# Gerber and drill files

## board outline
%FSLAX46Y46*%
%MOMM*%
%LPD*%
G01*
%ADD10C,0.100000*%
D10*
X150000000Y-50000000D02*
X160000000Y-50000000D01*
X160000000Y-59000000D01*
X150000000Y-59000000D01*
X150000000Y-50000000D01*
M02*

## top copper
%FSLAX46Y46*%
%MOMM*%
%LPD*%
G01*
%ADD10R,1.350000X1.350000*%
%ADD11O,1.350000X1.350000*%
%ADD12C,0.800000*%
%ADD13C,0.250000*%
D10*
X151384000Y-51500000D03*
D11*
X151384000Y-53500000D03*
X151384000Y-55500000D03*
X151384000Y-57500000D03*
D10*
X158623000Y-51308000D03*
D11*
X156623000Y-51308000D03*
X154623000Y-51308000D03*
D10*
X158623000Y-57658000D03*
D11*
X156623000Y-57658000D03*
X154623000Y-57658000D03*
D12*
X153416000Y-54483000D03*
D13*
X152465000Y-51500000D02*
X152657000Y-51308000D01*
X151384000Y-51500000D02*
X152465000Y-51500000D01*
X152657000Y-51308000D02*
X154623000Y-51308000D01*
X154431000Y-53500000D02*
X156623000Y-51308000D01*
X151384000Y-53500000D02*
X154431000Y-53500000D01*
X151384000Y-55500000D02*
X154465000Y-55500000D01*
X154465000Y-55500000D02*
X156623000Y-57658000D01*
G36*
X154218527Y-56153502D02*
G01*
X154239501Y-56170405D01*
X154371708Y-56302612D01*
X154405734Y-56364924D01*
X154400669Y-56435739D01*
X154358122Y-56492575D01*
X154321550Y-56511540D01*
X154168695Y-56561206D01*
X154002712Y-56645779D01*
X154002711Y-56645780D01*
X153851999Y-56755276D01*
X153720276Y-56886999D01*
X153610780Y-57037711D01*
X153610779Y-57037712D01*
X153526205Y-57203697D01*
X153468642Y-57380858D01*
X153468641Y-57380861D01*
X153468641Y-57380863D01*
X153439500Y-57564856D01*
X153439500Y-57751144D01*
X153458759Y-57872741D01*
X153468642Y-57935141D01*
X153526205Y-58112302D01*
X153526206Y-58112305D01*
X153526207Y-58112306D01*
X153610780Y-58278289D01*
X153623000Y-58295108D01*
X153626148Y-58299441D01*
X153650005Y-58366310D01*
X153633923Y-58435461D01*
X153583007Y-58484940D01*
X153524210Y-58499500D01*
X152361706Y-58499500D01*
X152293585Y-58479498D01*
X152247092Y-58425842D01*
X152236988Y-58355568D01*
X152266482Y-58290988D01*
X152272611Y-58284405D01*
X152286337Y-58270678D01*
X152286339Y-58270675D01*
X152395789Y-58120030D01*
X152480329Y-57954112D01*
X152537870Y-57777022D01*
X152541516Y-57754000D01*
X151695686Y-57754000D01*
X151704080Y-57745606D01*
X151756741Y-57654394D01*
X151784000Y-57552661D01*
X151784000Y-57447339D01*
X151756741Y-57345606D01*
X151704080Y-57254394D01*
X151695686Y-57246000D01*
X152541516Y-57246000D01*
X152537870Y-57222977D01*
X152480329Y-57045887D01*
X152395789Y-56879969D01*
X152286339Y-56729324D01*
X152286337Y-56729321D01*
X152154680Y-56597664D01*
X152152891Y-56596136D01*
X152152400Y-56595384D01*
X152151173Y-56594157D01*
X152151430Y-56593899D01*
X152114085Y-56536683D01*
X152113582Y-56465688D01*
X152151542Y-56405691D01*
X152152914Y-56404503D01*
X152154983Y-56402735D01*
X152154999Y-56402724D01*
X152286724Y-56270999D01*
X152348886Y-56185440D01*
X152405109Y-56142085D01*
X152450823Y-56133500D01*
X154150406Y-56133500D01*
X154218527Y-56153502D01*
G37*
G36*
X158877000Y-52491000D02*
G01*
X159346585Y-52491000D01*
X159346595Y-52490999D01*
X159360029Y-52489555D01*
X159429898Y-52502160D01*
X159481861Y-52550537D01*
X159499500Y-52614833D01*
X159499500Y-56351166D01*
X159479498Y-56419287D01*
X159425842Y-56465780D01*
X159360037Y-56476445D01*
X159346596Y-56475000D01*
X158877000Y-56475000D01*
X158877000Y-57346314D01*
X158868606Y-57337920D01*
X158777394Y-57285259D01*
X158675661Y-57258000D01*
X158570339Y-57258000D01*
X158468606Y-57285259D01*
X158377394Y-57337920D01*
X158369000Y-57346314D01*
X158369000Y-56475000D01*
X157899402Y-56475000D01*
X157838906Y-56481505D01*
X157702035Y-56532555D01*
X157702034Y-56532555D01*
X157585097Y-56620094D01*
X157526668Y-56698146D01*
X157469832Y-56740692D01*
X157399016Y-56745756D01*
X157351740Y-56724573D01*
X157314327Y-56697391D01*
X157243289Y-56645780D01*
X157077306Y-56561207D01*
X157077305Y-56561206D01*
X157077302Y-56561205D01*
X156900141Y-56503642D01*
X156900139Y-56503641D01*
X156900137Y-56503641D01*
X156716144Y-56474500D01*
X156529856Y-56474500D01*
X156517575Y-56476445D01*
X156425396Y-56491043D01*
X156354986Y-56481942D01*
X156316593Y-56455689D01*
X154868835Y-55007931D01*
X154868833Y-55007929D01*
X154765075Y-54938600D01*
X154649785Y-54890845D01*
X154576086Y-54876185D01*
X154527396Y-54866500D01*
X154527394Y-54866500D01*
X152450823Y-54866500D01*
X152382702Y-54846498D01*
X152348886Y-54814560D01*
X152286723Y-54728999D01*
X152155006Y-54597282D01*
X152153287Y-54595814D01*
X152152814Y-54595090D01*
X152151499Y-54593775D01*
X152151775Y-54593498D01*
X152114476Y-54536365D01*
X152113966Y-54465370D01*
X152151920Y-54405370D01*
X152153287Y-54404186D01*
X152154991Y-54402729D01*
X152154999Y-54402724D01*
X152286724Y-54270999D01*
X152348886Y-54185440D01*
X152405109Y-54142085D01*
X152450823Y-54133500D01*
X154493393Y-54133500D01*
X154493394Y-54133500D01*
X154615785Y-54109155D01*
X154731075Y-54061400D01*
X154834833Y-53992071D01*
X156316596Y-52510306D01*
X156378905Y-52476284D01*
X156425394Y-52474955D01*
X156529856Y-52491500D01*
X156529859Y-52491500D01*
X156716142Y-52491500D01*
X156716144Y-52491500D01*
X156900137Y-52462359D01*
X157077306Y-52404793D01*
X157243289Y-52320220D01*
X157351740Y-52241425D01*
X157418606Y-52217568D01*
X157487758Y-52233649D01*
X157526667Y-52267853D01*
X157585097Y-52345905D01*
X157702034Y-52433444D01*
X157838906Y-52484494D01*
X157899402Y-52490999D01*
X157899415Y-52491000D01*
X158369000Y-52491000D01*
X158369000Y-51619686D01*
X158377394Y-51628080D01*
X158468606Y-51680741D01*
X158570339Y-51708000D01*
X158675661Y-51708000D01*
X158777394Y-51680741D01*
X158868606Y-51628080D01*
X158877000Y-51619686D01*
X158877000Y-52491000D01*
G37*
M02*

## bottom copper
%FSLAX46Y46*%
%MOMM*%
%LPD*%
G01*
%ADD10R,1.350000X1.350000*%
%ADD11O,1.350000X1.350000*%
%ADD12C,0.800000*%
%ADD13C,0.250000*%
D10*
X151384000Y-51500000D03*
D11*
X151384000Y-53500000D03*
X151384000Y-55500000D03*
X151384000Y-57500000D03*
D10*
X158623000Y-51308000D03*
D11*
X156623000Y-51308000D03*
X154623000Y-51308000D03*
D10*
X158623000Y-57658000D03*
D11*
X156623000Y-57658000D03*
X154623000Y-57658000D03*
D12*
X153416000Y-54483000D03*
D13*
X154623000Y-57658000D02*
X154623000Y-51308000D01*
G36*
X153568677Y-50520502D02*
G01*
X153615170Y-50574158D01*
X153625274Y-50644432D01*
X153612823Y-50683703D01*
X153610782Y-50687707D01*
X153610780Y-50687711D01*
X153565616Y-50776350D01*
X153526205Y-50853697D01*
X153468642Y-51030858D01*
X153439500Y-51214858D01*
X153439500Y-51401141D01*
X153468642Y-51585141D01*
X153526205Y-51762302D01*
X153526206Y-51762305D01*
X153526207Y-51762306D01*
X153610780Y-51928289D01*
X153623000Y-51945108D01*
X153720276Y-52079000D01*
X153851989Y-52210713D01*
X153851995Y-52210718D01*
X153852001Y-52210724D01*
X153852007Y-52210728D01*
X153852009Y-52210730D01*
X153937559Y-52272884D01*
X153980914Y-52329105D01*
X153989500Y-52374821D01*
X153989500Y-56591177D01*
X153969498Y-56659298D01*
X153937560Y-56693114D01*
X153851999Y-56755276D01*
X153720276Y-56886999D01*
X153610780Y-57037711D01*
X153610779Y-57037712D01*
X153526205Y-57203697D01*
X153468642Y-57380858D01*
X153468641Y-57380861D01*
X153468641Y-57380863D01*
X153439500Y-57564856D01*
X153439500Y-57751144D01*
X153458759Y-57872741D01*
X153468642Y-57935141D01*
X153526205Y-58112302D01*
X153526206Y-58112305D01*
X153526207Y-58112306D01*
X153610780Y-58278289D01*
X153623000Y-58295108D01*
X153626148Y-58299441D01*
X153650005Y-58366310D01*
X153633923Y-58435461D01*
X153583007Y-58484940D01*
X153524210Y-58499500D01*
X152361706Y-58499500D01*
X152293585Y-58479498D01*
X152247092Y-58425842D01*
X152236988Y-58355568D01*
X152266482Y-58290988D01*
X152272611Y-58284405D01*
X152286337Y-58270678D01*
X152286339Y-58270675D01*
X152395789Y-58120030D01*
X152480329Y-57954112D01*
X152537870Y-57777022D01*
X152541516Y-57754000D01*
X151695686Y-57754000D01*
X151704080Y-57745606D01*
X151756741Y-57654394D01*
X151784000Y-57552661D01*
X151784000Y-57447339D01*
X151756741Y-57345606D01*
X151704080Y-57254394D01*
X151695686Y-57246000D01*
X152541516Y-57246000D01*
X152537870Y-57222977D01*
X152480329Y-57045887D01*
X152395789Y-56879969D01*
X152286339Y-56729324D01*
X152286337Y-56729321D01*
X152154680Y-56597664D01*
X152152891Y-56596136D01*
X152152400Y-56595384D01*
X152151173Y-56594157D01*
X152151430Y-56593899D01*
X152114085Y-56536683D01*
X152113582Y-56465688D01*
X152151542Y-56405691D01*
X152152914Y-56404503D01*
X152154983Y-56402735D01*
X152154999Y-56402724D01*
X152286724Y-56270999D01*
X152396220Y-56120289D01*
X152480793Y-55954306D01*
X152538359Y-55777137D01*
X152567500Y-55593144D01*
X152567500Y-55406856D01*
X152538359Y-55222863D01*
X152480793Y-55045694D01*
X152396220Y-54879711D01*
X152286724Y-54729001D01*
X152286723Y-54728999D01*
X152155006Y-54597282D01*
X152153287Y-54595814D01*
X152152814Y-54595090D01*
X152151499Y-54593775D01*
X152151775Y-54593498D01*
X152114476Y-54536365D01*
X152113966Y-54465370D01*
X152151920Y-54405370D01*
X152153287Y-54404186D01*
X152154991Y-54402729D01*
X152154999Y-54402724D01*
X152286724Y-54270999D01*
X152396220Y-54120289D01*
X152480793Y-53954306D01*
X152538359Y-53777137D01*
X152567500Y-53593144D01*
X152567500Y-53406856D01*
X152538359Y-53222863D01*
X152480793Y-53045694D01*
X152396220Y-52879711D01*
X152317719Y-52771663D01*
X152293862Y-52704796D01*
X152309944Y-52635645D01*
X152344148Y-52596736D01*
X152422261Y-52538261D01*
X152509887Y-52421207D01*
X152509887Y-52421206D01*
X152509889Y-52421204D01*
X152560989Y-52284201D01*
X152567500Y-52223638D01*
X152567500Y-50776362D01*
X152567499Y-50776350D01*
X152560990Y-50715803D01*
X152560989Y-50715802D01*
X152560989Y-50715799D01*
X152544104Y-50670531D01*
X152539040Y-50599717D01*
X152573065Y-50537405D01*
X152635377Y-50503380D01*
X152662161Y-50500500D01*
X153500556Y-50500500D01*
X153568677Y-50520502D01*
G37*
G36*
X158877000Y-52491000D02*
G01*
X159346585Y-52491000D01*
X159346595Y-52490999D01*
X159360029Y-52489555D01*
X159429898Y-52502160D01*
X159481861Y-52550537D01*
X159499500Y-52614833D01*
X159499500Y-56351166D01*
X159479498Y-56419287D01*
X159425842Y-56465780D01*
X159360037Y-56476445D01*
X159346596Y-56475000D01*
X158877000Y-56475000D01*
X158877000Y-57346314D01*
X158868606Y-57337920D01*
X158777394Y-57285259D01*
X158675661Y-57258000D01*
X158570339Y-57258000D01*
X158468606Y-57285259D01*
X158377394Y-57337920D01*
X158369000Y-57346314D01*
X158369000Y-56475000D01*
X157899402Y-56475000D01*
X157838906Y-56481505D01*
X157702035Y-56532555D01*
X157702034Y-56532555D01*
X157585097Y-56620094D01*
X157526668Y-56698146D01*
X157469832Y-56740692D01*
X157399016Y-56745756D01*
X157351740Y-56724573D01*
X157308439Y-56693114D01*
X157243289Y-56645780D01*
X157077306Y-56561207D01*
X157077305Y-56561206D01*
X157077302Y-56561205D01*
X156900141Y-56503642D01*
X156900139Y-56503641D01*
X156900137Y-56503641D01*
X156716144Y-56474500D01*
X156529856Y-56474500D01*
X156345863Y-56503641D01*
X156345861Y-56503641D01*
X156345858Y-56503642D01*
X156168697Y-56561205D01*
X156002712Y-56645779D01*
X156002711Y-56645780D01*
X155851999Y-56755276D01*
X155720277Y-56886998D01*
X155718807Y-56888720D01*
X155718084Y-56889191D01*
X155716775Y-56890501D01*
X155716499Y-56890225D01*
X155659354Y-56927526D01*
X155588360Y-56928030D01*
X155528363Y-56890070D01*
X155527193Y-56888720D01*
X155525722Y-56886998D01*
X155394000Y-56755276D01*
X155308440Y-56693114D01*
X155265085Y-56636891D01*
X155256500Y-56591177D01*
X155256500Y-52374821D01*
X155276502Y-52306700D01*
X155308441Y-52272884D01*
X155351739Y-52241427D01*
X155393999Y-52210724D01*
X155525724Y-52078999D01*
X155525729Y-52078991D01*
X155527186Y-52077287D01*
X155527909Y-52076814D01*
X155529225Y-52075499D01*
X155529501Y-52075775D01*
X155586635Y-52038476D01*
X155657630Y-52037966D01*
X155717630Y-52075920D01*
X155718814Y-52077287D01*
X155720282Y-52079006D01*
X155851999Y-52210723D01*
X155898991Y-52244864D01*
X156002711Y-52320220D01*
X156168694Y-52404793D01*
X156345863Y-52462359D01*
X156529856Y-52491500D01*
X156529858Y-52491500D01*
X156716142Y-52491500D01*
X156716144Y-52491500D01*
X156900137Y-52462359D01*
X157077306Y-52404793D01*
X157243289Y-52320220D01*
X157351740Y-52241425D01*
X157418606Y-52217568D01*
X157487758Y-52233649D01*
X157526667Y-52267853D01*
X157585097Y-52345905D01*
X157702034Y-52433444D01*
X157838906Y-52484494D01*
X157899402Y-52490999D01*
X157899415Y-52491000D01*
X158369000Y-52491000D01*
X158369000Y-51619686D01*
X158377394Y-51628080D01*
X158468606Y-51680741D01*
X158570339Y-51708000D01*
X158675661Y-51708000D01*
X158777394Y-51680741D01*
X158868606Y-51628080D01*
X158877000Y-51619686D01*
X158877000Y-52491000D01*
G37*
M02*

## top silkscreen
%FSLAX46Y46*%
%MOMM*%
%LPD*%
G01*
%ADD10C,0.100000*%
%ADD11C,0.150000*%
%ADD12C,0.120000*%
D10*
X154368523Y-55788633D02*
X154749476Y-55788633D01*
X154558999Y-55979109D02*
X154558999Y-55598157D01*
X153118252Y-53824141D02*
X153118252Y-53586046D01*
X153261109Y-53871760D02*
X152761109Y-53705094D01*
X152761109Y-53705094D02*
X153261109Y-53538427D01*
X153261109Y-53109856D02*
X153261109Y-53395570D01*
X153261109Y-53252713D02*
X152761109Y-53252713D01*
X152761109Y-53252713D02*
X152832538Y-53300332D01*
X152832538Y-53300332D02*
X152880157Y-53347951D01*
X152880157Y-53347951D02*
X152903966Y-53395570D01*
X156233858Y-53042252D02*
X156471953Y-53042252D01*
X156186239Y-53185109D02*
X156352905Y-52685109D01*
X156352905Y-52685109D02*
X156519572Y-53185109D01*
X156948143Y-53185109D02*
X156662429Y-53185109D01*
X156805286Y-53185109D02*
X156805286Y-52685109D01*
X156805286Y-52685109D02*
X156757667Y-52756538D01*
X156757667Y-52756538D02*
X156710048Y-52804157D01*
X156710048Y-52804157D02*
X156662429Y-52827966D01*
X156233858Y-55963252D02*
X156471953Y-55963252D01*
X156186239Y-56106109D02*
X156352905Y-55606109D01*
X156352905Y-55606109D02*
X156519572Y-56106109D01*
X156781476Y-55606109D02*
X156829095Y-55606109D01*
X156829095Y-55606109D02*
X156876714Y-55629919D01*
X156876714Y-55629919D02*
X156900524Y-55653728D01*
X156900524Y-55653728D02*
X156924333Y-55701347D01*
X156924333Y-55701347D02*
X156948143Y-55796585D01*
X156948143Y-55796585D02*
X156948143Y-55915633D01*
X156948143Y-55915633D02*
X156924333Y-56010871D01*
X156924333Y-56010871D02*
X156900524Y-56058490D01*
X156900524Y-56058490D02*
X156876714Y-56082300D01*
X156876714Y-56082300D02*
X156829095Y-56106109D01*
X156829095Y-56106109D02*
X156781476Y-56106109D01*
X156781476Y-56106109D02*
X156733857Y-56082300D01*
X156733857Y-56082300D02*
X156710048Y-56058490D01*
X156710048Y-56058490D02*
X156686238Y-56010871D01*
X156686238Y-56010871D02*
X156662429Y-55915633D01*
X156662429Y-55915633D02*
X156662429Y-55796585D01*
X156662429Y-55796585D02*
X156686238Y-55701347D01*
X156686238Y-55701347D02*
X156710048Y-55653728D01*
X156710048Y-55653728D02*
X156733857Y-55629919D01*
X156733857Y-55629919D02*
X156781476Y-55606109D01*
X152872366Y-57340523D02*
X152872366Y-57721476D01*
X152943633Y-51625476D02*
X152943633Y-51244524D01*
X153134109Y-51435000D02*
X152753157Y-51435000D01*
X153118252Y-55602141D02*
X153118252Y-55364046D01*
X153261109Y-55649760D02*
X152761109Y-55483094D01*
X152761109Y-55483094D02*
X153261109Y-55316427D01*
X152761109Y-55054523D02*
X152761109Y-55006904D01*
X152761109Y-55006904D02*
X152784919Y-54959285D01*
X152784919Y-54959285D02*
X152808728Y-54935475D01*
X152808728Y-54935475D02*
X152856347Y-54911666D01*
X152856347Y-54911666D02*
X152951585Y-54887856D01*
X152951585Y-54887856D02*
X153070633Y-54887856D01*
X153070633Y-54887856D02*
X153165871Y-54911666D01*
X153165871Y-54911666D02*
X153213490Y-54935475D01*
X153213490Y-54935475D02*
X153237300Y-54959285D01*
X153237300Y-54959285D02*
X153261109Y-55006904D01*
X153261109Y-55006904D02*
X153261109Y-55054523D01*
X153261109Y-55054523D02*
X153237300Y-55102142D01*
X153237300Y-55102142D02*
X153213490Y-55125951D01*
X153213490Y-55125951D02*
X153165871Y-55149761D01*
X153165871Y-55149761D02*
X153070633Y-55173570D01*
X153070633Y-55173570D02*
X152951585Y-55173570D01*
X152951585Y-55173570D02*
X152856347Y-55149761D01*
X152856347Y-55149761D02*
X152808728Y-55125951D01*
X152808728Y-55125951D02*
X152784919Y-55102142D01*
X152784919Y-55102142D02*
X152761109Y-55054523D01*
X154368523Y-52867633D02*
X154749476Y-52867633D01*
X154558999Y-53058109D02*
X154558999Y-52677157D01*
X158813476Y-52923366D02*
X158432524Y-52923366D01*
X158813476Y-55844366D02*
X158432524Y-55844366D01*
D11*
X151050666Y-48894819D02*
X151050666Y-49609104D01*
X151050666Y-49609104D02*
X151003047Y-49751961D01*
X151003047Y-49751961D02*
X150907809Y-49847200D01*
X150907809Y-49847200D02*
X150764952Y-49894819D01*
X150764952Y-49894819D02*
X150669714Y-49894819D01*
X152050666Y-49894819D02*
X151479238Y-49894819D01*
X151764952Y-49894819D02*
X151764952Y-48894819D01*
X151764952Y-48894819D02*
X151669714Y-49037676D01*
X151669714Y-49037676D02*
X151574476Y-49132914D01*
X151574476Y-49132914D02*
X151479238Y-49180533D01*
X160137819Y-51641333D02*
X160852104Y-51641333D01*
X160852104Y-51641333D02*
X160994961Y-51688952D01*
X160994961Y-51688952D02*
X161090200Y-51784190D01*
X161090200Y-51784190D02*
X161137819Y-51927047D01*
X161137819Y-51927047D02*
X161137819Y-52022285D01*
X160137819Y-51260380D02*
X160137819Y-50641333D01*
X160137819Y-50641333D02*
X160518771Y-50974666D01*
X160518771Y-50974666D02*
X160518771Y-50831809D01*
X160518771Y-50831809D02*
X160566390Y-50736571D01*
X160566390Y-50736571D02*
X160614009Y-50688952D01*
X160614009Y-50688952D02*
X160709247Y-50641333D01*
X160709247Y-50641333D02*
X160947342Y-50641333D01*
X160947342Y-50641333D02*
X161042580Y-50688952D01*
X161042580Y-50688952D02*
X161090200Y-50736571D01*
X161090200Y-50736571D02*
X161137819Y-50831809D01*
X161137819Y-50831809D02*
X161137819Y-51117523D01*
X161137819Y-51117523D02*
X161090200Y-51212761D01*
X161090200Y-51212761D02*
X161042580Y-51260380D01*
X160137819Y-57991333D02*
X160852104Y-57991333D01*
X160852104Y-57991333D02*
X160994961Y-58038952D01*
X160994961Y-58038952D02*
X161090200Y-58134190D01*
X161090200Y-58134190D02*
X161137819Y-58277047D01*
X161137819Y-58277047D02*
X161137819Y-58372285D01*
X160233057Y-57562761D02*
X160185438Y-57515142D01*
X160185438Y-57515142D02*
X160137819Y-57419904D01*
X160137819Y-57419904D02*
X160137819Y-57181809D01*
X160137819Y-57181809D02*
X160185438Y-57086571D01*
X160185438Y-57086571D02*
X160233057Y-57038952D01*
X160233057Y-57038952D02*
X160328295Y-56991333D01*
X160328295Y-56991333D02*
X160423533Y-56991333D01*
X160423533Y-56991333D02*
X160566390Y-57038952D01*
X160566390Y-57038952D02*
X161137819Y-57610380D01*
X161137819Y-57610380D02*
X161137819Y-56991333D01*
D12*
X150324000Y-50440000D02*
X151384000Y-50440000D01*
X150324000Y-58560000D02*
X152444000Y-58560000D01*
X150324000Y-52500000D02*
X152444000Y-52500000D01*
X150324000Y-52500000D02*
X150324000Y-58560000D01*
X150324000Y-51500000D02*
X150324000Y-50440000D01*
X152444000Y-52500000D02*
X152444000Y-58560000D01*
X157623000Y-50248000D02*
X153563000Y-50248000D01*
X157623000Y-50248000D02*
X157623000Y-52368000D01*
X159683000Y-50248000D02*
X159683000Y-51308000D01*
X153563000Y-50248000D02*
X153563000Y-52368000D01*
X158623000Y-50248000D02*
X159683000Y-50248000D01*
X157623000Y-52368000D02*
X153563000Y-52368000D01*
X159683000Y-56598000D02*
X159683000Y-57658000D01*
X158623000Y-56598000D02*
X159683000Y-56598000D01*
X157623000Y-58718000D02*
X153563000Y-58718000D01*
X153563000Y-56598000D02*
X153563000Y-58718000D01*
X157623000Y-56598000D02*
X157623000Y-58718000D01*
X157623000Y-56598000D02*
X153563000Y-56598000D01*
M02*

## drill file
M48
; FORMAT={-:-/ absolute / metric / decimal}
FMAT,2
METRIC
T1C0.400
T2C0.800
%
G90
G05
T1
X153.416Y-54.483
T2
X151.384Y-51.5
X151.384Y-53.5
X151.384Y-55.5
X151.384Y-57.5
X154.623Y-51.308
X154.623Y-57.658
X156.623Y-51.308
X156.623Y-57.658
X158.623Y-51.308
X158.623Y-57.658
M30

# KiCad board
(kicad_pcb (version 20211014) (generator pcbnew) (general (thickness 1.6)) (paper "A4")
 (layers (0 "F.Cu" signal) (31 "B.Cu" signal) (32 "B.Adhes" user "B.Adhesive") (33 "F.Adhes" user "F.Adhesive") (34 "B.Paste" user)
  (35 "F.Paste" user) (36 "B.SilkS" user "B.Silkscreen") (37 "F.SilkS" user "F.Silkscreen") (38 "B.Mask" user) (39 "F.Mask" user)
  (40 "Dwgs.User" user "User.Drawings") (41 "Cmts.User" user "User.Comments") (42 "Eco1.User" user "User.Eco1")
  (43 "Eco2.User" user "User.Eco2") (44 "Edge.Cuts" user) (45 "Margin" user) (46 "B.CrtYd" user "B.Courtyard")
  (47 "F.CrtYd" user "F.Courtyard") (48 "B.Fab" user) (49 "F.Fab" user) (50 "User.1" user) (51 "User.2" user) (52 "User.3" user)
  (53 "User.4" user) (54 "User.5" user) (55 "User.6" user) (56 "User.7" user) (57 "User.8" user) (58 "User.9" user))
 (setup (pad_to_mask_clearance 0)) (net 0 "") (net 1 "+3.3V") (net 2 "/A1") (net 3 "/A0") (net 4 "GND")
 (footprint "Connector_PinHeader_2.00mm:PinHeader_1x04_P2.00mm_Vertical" (layer "F.Cu") (at 151.384 51.5)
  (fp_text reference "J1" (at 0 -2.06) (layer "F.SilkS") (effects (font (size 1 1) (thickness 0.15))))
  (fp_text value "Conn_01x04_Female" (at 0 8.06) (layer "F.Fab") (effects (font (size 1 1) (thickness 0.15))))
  (fp_line (start -1.06 -1.06) (end 0 -1.06) (layer "F.SilkS") (width 0.12))
  (fp_line (start -1.06 7.06) (end 1.06 7.06) (layer "F.SilkS") (width 0.12))
  (fp_line (start -1.06 1) (end 1.06 1) (layer "F.SilkS") (width 0.12))
  (fp_line (start -1.06 1) (end -1.06 7.06) (layer "F.SilkS") (width 0.12))
  (fp_line (start -1.06 0) (end -1.06 -1.06) (layer "F.SilkS") (width 0.12))
  (fp_line (start 1.06 1) (end 1.06 7.06) (layer "F.SilkS") (width 0.12))
  (pad "1" thru_hole rect (at 0 0) (size 1.35 1.35) (drill 0.8) (layers *.Cu *.Mask) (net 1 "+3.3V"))
  (pad "2" thru_hole oval (at 0 2) (size 1.35 1.35) (drill 0.8) (layers *.Cu *.Mask) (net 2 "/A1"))
  (pad "3" thru_hole oval (at 0 4) (size 1.35 1.35) (drill 0.8) (layers *.Cu *.Mask) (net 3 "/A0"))
  (pad "4" thru_hole oval (at 0 6) (size 1.35 1.35) (drill 0.8) (layers *.Cu *.Mask) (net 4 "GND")))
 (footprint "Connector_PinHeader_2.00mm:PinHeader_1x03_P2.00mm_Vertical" (layer "F.Cu") (at 158.623 51.308 -90)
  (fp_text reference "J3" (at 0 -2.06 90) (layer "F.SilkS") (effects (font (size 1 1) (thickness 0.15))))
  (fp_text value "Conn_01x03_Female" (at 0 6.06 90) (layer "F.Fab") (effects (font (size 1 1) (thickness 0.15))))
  (fp_line (start -1.06 1) (end -1.06 5.06) (layer "F.SilkS") (width 0.12))
  (fp_line (start -1.06 1) (end 1.06 1) (layer "F.SilkS") (width 0.12))
  (fp_line (start -1.06 -1.06) (end 0 -1.06) (layer "F.SilkS") (width 0.12))
  (fp_line (start -1.06 5.06) (end 1.06 5.06) (layer "F.SilkS") (width 0.12))
  (fp_line (start -1.06 0) (end -1.06 -1.06) (layer "F.SilkS") (width 0.12))
  (fp_line (start 1.06 1) (end 1.06 5.06) (layer "F.SilkS") (width 0.12))
  (pad "1" thru_hole rect (at 0 0 270) (size 1.35 1.35) (drill 0.8) (layers *.Cu *.Mask) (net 4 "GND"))
  (pad "2" thru_hole oval (at 0 2 270) (size 1.35 1.35) (drill 0.8) (layers *.Cu *.Mask) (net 2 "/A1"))
  (pad "3" thru_hole oval (at 0 4 270) (size 1.35 1.35) (drill 0.8) (layers *.Cu *.Mask) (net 1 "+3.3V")))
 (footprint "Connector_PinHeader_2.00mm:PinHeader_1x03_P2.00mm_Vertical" (layer "F.Cu") (at 158.623 57.658 -90)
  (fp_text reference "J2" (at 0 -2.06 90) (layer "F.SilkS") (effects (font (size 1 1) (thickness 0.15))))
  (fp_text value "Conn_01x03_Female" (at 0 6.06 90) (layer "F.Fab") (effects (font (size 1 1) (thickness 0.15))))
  (fp_line (start -1.06 -1.06) (end 0 -1.06) (layer "F.SilkS") (width 0.12))
  (fp_line (start -1.06 0) (end -1.06 -1.06) (layer "F.SilkS") (width 0.12))
  (fp_line (start 1.06 1) (end 1.06 5.06) (layer "F.SilkS") (width 0.12))
  (fp_line (start -1.06 5.06) (end 1.06 5.06) (layer "F.SilkS") (width 0.12))
  (fp_line (start -1.06 1) (end 1.06 1) (layer "F.SilkS") (width 0.12))
  (fp_line (start -1.06 1) (end -1.06 5.06) (layer "F.SilkS") (width 0.12))
  (pad "1" thru_hole rect (at 0 0 270) (size 1.35 1.35) (drill 0.8) (layers *.Cu *.Mask) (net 4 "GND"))
  (pad "2" thru_hole oval (at 0 2 270) (size 1.35 1.35) (drill 0.8) (layers *.Cu *.Mask) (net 3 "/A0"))
  (pad "3" thru_hole oval (at 0 4 270) (size 1.35 1.35) (drill 0.8) (layers *.Cu *.Mask) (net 1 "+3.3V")))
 (gr_rect (start 150 50) (end 160 59) (layer "Edge.Cuts") (width 0.1) (fill none))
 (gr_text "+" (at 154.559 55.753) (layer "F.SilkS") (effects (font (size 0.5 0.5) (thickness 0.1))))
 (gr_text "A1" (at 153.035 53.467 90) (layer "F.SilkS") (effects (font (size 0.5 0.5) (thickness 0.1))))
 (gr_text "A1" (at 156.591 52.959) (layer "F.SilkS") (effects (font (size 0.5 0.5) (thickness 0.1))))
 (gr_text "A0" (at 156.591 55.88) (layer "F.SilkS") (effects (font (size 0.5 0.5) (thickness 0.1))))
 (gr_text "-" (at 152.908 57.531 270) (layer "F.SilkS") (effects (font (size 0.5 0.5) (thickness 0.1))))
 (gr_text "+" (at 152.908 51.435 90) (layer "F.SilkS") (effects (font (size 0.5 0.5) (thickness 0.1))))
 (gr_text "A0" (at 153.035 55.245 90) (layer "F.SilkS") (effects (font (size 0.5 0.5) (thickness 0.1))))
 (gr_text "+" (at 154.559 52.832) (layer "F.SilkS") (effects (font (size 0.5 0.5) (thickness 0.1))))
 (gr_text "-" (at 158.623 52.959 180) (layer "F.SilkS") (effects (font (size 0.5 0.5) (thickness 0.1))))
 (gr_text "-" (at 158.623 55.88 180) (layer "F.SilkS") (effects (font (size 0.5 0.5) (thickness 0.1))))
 (segment (start 152.465 51.5) (end 152.657 51.308) (width 0.25) (layer "F.Cu") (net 1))
 (segment (start 151.384 51.5) (end 152.465 51.5) (width 0.25) (layer "F.Cu") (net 1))
 (segment (start 152.657 51.308) (end 154.623 51.308) (width 0.25) (layer "F.Cu") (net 1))
 (segment (start 154.623 57.658) (end 154.623 51.308) (width 0.25) (layer "B.Cu") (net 1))
 (segment (start 154.431 53.5) (end 156.623 51.308) (width 0.25) (layer "F.Cu") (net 2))
 (segment (start 151.384 53.5) (end 154.431 53.5) (width 0.25) (layer "F.Cu") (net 2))
 (segment (start 151.384 55.5) (end 154.465 55.5) (width 0.25) (layer "F.Cu") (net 3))
 (segment (start 154.465 55.5) (end 156.623 57.658) (width 0.25) (layer "F.Cu") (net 3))
 (via (at 153.416 54.483) (size 0.8) (drill 0.4) (layers "F.Cu" "B.Cu") (free) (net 4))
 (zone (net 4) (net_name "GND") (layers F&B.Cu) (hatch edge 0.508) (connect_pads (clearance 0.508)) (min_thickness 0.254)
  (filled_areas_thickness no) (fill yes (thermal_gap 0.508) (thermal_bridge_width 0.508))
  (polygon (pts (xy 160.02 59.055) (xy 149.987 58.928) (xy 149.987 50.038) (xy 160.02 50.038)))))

